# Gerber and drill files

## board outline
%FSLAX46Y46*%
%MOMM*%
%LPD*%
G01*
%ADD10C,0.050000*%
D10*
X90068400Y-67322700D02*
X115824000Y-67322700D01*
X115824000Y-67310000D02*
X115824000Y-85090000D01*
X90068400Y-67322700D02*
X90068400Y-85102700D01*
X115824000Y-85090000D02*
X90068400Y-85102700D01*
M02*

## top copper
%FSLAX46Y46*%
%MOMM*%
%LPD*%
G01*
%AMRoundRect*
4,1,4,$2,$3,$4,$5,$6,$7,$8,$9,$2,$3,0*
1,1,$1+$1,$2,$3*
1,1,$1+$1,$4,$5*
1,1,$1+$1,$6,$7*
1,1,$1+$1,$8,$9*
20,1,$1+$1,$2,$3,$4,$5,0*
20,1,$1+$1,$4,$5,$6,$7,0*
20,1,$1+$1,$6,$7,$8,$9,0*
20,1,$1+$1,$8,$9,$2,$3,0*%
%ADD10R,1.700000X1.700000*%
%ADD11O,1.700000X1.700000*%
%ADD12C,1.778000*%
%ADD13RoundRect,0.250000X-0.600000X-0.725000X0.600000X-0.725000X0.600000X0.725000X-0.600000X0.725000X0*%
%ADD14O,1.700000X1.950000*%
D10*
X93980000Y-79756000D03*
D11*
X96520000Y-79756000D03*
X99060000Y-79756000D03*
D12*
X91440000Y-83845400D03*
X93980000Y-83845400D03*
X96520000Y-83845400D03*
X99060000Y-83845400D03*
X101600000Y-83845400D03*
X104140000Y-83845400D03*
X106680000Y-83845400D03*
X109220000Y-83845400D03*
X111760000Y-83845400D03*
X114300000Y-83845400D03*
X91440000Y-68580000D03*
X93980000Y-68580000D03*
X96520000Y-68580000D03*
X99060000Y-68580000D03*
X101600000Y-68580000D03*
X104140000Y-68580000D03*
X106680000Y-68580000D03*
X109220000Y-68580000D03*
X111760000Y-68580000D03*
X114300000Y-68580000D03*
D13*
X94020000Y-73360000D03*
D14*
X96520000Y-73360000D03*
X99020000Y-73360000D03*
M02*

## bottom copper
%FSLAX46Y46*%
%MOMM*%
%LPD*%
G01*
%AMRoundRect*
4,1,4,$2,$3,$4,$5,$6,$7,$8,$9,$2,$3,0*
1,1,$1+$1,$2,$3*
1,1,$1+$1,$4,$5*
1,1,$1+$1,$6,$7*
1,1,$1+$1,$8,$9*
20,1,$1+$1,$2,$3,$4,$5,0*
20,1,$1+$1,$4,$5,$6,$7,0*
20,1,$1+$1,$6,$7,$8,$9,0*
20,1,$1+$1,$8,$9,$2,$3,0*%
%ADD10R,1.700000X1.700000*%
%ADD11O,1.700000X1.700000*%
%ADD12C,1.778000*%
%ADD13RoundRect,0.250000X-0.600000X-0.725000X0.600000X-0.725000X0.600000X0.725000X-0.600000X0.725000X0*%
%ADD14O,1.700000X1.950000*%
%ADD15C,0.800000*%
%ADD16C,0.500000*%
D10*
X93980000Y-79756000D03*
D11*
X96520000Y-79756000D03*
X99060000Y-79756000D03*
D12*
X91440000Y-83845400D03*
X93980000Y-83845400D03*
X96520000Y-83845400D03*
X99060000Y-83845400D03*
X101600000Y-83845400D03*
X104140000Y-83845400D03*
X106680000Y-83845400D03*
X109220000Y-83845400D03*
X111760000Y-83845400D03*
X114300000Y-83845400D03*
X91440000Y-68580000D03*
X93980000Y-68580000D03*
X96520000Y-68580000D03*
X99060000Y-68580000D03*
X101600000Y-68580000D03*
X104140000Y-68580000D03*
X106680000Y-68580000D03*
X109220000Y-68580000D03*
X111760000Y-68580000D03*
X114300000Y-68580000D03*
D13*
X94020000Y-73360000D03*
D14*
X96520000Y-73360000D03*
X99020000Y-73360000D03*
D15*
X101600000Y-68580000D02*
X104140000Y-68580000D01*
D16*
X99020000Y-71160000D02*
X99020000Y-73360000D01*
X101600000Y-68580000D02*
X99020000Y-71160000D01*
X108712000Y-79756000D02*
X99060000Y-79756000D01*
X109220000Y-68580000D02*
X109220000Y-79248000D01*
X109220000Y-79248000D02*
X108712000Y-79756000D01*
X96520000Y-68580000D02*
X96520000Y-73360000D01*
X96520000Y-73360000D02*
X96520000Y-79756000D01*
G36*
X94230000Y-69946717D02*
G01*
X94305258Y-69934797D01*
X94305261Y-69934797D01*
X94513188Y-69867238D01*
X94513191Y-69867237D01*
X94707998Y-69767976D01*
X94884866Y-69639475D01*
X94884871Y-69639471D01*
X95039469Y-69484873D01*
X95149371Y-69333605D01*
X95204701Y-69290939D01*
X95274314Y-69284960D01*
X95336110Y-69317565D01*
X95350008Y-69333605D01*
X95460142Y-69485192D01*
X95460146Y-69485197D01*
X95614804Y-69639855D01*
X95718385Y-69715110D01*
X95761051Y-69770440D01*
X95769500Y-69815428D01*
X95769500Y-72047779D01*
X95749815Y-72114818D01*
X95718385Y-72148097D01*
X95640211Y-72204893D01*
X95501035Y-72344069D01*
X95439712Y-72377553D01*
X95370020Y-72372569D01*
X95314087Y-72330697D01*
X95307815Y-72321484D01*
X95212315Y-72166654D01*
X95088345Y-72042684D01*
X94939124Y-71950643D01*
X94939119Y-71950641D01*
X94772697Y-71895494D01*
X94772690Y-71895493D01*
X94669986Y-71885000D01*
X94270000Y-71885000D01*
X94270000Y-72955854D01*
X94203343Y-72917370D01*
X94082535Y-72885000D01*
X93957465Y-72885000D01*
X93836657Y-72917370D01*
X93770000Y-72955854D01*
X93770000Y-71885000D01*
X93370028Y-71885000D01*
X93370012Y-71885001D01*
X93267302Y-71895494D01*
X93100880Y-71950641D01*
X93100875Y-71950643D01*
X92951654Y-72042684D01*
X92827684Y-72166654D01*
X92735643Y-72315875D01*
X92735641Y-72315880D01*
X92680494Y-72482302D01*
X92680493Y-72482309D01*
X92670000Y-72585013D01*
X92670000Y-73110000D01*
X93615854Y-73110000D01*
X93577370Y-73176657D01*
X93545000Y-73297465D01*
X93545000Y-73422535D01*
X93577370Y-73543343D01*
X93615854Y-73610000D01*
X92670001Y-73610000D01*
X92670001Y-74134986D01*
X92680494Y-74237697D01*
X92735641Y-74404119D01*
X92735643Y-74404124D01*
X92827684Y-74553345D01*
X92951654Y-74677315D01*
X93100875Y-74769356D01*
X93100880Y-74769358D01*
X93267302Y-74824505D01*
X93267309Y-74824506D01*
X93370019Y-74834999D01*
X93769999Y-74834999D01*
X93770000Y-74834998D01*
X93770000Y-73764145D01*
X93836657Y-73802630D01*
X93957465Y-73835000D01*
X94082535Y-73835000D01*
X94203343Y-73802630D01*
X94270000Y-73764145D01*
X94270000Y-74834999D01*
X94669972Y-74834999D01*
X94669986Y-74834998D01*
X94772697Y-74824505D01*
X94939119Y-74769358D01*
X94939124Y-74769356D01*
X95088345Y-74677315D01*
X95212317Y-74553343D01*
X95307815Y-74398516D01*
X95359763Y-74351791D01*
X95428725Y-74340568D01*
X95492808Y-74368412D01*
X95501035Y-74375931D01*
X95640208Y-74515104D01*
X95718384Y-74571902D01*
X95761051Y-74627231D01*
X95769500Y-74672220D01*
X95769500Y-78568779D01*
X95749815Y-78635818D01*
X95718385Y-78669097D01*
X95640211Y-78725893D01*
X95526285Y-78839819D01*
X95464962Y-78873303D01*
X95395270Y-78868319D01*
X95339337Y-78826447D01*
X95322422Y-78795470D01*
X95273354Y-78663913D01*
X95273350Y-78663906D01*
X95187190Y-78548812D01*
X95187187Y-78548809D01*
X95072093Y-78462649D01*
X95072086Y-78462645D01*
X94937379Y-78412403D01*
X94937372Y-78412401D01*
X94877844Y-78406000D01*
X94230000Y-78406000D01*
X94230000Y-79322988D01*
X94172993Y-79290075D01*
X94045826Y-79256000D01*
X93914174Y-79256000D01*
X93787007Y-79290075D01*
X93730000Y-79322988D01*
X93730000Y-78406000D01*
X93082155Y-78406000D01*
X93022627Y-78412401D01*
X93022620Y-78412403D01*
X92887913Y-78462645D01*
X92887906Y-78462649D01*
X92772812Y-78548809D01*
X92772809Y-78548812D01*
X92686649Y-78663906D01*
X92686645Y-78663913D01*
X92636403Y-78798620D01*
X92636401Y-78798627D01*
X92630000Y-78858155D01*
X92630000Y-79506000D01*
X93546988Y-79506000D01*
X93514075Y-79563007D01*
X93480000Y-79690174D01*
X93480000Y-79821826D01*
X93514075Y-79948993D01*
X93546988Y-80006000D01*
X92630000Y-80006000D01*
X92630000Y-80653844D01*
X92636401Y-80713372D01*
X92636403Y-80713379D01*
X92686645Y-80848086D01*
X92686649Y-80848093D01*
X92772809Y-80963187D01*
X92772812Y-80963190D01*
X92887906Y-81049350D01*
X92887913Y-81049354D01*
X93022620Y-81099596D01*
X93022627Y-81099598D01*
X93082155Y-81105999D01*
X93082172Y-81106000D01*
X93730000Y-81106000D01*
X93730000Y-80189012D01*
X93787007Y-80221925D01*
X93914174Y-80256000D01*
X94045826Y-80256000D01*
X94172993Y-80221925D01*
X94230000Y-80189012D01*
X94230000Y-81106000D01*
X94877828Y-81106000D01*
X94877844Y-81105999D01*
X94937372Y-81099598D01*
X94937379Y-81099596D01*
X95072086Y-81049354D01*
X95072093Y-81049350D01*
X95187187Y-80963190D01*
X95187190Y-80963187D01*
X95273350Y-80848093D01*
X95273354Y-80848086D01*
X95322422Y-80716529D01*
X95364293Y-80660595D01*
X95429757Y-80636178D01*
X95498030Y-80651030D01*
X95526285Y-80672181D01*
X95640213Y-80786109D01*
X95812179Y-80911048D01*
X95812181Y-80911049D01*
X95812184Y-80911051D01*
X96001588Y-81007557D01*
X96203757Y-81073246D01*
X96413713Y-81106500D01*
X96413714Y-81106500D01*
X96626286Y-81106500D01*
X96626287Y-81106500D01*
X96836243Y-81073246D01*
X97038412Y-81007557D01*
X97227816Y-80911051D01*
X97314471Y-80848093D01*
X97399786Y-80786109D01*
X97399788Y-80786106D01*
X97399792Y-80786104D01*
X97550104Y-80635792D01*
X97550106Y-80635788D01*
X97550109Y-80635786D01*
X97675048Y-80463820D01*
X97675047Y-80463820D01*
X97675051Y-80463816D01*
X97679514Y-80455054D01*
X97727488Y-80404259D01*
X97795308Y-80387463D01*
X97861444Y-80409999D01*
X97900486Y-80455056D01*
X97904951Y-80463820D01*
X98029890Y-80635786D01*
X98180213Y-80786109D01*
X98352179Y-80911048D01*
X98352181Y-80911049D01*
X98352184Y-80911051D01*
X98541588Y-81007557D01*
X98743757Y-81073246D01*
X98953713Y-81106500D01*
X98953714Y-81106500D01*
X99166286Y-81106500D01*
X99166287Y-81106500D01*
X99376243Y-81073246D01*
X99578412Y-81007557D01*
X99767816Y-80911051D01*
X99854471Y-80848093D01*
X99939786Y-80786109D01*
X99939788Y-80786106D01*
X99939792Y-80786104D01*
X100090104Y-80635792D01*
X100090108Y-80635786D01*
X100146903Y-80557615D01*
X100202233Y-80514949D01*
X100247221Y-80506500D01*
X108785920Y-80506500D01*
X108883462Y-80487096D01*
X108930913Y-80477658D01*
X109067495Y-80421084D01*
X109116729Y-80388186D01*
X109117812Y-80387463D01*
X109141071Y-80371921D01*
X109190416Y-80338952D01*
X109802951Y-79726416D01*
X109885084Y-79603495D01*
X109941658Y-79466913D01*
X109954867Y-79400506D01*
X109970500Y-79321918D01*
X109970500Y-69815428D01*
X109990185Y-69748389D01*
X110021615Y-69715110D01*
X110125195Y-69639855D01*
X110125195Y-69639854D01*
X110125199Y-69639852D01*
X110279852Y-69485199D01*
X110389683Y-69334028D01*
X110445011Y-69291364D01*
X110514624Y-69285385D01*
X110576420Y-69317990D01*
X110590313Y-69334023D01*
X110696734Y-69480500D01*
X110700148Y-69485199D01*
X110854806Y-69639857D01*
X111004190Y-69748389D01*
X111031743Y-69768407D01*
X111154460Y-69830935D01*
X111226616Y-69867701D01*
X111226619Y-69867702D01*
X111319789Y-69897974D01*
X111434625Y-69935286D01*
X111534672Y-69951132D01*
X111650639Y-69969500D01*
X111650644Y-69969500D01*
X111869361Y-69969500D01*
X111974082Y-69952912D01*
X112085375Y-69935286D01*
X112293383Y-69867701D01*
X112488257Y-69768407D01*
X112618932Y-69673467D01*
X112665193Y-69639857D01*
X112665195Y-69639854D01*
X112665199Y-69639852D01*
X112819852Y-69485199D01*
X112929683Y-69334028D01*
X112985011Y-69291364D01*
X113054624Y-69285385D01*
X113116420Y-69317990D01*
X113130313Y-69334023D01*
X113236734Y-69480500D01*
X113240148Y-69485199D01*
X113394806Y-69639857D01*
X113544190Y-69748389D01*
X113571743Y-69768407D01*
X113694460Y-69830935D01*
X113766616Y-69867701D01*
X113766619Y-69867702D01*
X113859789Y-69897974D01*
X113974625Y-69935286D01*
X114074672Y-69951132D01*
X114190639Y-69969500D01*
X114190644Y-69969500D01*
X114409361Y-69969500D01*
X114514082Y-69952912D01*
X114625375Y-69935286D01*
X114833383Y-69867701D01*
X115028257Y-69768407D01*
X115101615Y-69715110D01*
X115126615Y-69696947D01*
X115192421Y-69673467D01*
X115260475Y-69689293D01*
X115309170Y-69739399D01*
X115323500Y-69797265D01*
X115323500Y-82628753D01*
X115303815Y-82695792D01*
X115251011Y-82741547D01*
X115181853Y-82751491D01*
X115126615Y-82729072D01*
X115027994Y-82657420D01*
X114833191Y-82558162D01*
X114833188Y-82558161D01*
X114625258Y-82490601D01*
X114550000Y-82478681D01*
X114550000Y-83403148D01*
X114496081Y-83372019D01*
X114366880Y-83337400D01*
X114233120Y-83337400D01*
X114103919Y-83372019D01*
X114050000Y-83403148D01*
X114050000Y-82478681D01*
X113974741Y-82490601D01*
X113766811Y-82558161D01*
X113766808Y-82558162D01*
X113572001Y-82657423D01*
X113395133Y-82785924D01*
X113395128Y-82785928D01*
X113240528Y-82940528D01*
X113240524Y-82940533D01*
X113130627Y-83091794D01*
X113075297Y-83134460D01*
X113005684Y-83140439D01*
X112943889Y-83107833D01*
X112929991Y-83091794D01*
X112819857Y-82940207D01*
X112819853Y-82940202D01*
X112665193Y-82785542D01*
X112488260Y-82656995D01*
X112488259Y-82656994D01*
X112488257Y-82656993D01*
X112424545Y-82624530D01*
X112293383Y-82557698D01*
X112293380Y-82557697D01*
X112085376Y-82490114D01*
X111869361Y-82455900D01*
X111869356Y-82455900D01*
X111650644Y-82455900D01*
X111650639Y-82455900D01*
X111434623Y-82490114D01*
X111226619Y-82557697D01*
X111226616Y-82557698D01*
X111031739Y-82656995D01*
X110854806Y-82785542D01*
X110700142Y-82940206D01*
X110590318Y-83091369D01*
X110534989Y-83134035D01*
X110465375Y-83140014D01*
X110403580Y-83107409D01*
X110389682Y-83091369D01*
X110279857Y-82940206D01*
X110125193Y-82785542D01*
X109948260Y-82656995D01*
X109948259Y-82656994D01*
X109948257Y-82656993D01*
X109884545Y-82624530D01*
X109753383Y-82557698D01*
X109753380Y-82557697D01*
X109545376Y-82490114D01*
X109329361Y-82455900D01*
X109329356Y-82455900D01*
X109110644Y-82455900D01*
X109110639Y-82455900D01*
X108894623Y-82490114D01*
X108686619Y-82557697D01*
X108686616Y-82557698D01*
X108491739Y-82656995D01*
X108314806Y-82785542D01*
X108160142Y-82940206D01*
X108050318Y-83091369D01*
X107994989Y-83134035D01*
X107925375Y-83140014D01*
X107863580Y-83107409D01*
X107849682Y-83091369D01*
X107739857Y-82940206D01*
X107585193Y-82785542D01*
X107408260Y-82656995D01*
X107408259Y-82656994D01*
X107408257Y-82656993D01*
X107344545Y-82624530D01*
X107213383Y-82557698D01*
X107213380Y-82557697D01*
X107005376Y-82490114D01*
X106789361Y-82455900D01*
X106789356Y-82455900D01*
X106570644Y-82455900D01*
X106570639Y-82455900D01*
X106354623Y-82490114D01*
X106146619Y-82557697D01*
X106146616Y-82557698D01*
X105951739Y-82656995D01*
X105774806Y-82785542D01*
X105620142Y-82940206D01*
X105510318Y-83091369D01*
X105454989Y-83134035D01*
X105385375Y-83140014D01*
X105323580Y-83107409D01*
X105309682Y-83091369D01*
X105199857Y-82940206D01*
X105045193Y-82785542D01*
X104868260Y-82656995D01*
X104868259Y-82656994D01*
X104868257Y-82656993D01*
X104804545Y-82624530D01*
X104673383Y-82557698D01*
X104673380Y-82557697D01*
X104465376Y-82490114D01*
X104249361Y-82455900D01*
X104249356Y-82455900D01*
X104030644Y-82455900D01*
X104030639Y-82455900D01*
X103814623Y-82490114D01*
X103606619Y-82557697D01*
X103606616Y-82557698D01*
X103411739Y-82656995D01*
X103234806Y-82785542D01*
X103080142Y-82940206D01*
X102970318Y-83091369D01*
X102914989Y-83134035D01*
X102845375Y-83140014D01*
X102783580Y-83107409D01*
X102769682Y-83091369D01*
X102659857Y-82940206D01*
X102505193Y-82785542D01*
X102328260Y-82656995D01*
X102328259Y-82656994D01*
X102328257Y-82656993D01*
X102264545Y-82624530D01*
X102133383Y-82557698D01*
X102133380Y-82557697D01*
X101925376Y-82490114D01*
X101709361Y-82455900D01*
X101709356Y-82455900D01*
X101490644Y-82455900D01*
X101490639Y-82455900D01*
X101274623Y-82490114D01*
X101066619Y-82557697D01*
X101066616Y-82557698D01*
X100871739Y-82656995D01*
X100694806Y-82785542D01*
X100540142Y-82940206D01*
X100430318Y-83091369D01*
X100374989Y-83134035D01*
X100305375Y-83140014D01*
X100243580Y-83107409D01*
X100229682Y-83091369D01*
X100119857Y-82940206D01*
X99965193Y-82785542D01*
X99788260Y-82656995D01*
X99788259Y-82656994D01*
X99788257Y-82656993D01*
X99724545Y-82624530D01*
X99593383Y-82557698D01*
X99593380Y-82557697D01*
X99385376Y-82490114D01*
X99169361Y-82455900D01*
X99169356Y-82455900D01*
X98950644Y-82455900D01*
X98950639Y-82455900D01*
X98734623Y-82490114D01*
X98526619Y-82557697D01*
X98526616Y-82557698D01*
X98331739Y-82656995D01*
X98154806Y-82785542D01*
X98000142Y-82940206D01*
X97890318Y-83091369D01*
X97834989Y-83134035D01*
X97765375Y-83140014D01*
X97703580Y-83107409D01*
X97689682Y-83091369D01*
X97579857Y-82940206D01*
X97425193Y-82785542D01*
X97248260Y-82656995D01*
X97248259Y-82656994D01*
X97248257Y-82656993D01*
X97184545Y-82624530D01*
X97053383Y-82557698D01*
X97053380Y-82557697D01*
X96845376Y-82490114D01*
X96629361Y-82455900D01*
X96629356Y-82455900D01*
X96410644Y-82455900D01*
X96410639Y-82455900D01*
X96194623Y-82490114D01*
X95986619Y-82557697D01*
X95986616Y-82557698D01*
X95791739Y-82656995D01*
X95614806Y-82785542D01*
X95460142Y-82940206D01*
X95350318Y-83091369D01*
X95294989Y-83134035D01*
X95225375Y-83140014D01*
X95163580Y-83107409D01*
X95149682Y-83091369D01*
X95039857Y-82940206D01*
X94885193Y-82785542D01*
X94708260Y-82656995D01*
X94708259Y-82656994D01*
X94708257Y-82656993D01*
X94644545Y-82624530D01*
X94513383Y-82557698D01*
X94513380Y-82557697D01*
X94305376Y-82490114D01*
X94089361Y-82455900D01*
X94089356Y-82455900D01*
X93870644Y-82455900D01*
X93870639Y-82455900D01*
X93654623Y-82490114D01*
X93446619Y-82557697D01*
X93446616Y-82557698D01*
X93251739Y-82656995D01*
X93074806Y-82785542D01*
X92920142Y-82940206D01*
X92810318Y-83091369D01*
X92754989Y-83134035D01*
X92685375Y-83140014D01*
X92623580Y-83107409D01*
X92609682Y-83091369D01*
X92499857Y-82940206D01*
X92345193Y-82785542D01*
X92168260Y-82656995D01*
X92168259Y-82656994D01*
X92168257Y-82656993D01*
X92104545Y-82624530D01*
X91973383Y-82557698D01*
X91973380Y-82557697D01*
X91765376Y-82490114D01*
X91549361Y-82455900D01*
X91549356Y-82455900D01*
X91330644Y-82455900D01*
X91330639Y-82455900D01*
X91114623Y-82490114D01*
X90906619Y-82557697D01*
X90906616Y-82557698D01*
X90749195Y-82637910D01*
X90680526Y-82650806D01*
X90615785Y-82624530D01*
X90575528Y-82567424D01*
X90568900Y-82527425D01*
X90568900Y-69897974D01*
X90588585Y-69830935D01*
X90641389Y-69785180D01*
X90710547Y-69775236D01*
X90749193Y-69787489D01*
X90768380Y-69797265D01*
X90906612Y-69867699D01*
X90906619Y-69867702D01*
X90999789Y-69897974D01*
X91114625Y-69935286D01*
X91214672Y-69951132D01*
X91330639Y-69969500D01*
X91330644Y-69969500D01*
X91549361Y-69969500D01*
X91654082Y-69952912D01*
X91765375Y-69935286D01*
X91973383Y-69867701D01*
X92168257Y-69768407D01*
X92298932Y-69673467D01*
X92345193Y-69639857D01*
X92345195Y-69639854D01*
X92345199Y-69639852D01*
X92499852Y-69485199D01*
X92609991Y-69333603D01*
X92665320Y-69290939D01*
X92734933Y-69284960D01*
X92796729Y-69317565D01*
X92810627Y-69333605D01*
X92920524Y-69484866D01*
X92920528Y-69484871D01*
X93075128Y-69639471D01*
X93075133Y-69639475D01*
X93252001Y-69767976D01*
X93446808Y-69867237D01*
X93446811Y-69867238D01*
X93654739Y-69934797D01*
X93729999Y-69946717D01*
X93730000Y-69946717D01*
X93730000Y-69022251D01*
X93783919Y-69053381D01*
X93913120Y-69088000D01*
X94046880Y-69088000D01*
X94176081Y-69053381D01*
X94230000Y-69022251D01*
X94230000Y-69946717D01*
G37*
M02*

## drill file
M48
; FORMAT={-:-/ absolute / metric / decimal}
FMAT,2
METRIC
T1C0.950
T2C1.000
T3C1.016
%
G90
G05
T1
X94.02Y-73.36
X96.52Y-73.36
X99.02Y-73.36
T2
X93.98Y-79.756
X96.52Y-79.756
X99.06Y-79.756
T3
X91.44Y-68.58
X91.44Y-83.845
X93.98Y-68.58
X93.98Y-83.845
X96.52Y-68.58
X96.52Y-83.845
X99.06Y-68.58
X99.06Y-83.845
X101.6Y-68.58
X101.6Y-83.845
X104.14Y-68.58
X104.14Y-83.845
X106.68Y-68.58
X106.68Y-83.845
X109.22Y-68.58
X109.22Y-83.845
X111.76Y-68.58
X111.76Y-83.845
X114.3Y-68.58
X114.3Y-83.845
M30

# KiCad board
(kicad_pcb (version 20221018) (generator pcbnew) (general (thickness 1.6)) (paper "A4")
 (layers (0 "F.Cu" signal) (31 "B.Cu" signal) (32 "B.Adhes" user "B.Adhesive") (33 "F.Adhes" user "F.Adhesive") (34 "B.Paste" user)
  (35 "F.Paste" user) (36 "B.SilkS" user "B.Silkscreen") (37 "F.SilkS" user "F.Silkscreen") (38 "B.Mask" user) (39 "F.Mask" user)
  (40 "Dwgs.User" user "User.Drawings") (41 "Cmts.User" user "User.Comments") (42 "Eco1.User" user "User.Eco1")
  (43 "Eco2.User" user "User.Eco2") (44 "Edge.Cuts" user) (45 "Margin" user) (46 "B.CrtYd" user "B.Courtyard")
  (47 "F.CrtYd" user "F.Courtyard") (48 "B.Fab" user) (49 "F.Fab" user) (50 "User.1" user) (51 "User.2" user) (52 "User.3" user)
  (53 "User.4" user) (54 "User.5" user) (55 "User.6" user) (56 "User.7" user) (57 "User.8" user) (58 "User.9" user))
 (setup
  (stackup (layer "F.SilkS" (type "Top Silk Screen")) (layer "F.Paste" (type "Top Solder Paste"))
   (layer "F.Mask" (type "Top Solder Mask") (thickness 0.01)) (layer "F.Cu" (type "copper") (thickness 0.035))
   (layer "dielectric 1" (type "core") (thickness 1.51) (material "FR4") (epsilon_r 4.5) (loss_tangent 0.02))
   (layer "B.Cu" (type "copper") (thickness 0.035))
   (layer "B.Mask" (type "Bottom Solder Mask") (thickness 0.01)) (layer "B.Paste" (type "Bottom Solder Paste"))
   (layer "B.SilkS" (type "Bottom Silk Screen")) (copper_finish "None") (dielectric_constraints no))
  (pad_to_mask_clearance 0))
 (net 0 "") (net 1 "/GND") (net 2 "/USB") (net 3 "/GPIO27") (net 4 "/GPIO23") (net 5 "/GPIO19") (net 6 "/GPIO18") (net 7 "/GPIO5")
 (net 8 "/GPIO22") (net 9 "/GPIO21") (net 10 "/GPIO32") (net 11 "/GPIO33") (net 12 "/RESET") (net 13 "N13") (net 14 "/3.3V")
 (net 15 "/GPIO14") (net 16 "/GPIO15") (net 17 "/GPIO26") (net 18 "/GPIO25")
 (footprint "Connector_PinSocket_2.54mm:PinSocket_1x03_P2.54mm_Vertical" (layer "F.Cu") (at 93.98 79.756 90)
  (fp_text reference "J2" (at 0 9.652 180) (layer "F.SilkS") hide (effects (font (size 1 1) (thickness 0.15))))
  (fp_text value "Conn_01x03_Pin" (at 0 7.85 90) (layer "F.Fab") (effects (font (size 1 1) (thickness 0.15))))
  (pad "1" thru_hole rect (at 0 0 90) (size 1.7 1.7) (drill 1) (layers "*.Cu" "*.Mask") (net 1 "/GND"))
  (pad "2" thru_hole oval (at 0 2.54 90) (size 1.7 1.7) (drill 1) (layers "*.Cu" "*.Mask") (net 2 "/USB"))
  (pad "3" thru_hole oval (at 0 5.08 90) (size 1.7 1.7) (drill 1) (layers "*.Cu" "*.Mask") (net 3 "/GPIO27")))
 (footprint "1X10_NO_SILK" (layer "F.Cu") (at 91.44 83.8454)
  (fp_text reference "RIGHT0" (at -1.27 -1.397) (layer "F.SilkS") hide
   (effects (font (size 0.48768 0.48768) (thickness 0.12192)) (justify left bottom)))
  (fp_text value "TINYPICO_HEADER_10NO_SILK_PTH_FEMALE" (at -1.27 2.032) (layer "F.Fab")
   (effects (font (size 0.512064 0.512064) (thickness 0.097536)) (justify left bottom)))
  (pad "1" thru_hole circle (at 0 0 90) (size 1.778 1.778) (drill 1.016) (layers "*.Cu" "*.Mask") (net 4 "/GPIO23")
   (solder_mask_margin 0.1016) (thermal_bridge_angle 0))
  (pad "2" thru_hole circle (at 2.54 0 90) (size 1.778 1.778) (drill 1.016) (layers "*.Cu" "*.Mask") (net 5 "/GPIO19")
   (solder_mask_margin 0.1016) (thermal_bridge_angle 0))
  (pad "3" thru_hole circle (at 5.08 0 90) (size 1.778 1.778) (drill 1.016) (layers "*.Cu" "*.Mask") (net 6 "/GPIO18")
   (solder_mask_margin 0.1016) (thermal_bridge_angle 0))
  (pad "4" thru_hole circle (at 7.62 0 90) (size 1.778 1.778) (drill 1.016) (layers "*.Cu" "*.Mask") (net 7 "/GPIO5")
   (solder_mask_margin 0.1016) (thermal_bridge_angle 0))
  (pad "5" thru_hole circle (at 10.16 0 90) (size 1.778 1.778) (drill 1.016) (layers "*.Cu" "*.Mask") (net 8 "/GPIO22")
   (solder_mask_margin 0.1016) (thermal_bridge_angle 0))
  (pad "6" thru_hole circle (at 12.7 0 90) (size 1.778 1.778) (drill 1.016) (layers "*.Cu" "*.Mask") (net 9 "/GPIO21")
   (solder_mask_margin 0.1016) (thermal_bridge_angle 0))
  (pad "7" thru_hole circle (at 15.24 0 90) (size 1.778 1.778) (drill 1.016) (layers "*.Cu" "*.Mask") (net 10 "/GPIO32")
   (solder_mask_margin 0.1016) (thermal_bridge_angle 0))
  (pad "8" thru_hole circle (at 17.78 0 90) (size 1.778 1.778) (drill 1.016) (layers "*.Cu" "*.Mask") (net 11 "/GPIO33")
   (solder_mask_margin 0.1016) (thermal_bridge_angle 0))
  (pad "9" thru_hole circle (at 20.32 0 90) (size 1.778 1.778) (drill 1.016) (layers "*.Cu" "*.Mask") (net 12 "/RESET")
   (solder_mask_margin 0.1016) (thermal_bridge_angle 0))
  (pad "10" thru_hole circle (at 22.86 0 90) (size 1.778 1.778) (drill 1.016) (layers "*.Cu" "*.Mask") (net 1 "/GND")
   (solder_mask_margin 0.1016) (thermal_bridge_angle 0)))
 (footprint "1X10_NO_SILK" (layer "F.Cu") (at 91.44 68.58)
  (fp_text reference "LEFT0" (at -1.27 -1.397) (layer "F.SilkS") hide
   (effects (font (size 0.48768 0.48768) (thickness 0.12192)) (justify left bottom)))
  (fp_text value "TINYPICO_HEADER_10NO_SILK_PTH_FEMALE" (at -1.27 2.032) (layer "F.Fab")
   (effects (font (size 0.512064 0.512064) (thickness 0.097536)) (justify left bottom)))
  (pad "1" thru_hole circle (at 0 0 90) (size 1.778 1.778) (drill 1.016) (layers "*.Cu" "*.Mask") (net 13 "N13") (solder_mask_margin 0.1016)
   (thermal_bridge_angle 0))
  (pad "2" thru_hole circle (at 2.54 0 90) (size 1.778 1.778) (drill 1.016) (layers "*.Cu" "*.Mask") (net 1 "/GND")
   (solder_mask_margin 0.1016) (thermal_bridge_angle 0))
  (pad "3" thru_hole circle (at 5.08 0 90) (size 1.778 1.778) (drill 1.016) (layers "*.Cu" "*.Mask") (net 2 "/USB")
   (solder_mask_margin 0.1016) (thermal_bridge_angle 0))
  (pad "4" thru_hole circle (at 7.62 0 90) (size 1.778 1.778) (drill 1.016) (layers "*.Cu" "*.Mask") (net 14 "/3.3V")
   (solder_mask_margin 0.1016) (thermal_bridge_angle 0))
  (pad "5" thru_hole circle (at 10.16 0 90) (size 1.778 1.778) (drill 1.016) (layers "*.Cu" "*.Mask") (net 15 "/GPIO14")
   (solder_mask_margin 0.1016) (thermal_bridge_angle 0))
  (pad "6" thru_hole circle (at 12.7 0 90) (size 1.778 1.778) (drill 1.016) (layers "*.Cu" "*.Mask") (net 15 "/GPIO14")
   (solder_mask_margin 0.1016) (thermal_bridge_angle 0))
  (pad "7" thru_hole circle (at 15.24 0 90) (size 1.778 1.778) (drill 1.016) (layers "*.Cu" "*.Mask") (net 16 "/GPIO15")
   (solder_mask_margin 0.1016) (thermal_bridge_angle 0))
  (pad "8" thru_hole circle (at 17.78 0 90) (size 1.778 1.778) (drill 1.016) (layers "*.Cu" "*.Mask") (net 3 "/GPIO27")
   (solder_mask_margin 0.1016) (thermal_bridge_angle 0))
  (pad "9" thru_hole circle (at 20.32 0 90) (size 1.778 1.778) (drill 1.016) (layers "*.Cu" "*.Mask") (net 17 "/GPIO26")
   (solder_mask_margin 0.1016) (thermal_bridge_angle 0))
  (pad "10" thru_hole circle (at 22.86 0 90) (size 1.778 1.778) (drill 1.016) (layers "*.Cu" "*.Mask") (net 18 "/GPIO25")
   (solder_mask_margin 0.1016) (thermal_bridge_angle 0)))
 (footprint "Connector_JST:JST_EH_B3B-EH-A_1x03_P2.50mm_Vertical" (layer "F.Cu") (at 94.02 73.36)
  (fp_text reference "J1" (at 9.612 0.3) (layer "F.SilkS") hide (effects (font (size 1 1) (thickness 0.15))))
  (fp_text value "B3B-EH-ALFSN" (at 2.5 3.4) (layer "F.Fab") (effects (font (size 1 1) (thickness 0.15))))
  (pad "1" thru_hole roundrect (at 0 0) (size 1.7 1.95) (drill 0.95) (layers "*.Cu" "*.Mask") (roundrect_rratio 0.1470588235) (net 1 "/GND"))
  (pad "2" thru_hole oval (at 2.5 0) (size 1.7 1.95) (drill 0.95) (layers "*.Cu" "*.Mask") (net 2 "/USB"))
  (pad "3" thru_hole oval (at 5 0) (size 1.7 1.95) (drill 0.95) (layers "*.Cu" "*.Mask") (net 15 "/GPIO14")))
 (gr_line (start 90.0684 67.3227) (end 115.824 67.3227) (stroke (width 0.05) (type solid)) (layer "Edge.Cuts"))
 (gr_line (start 115.824 67.31) (end 115.824 85.09) (stroke (width 0.05) (type solid)) (layer "Edge.Cuts"))
 (gr_line (start 90.0684 67.3227) (end 90.0684 85.1027) (stroke (width 0.05) (type solid)) (layer "Edge.Cuts"))
 (gr_line (start 115.824 85.09) (end 90.0684 85.1027) (stroke (width 0.05) (type solid)) (layer "Edge.Cuts"))
 (segment (start 101.6 68.58) (end 104.14 68.58) (width 0.8) (layer "B.Cu") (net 15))
 (segment (start 99.02 71.16) (end 99.02 73.36) (width 0.5) (layer "B.Cu") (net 15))
 (segment (start 101.6 68.58) (end 99.02 71.16) (width 0.5) (layer "B.Cu") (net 15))
 (segment (start 108.712 79.756) (end 99.06 79.756) (width 0.5) (layer "B.Cu") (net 3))
 (segment (start 109.22 68.58) (end 109.22 79.248) (width 0.5) (layer "B.Cu") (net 3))
 (segment (start 109.22 79.248) (end 108.712 79.756) (width 0.5) (layer "B.Cu") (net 3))
 (segment (start 96.52 68.58) (end 96.52 73.36) (width 0.5) (layer "B.Cu") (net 2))
 (segment (start 96.52 73.36) (end 96.52 79.756) (width 0.5) (layer "B.Cu") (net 2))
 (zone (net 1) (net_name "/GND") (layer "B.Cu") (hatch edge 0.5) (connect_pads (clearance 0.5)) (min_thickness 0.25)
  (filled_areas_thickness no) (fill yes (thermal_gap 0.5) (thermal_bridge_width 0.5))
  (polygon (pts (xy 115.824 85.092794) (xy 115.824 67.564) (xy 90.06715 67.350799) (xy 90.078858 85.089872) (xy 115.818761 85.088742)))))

